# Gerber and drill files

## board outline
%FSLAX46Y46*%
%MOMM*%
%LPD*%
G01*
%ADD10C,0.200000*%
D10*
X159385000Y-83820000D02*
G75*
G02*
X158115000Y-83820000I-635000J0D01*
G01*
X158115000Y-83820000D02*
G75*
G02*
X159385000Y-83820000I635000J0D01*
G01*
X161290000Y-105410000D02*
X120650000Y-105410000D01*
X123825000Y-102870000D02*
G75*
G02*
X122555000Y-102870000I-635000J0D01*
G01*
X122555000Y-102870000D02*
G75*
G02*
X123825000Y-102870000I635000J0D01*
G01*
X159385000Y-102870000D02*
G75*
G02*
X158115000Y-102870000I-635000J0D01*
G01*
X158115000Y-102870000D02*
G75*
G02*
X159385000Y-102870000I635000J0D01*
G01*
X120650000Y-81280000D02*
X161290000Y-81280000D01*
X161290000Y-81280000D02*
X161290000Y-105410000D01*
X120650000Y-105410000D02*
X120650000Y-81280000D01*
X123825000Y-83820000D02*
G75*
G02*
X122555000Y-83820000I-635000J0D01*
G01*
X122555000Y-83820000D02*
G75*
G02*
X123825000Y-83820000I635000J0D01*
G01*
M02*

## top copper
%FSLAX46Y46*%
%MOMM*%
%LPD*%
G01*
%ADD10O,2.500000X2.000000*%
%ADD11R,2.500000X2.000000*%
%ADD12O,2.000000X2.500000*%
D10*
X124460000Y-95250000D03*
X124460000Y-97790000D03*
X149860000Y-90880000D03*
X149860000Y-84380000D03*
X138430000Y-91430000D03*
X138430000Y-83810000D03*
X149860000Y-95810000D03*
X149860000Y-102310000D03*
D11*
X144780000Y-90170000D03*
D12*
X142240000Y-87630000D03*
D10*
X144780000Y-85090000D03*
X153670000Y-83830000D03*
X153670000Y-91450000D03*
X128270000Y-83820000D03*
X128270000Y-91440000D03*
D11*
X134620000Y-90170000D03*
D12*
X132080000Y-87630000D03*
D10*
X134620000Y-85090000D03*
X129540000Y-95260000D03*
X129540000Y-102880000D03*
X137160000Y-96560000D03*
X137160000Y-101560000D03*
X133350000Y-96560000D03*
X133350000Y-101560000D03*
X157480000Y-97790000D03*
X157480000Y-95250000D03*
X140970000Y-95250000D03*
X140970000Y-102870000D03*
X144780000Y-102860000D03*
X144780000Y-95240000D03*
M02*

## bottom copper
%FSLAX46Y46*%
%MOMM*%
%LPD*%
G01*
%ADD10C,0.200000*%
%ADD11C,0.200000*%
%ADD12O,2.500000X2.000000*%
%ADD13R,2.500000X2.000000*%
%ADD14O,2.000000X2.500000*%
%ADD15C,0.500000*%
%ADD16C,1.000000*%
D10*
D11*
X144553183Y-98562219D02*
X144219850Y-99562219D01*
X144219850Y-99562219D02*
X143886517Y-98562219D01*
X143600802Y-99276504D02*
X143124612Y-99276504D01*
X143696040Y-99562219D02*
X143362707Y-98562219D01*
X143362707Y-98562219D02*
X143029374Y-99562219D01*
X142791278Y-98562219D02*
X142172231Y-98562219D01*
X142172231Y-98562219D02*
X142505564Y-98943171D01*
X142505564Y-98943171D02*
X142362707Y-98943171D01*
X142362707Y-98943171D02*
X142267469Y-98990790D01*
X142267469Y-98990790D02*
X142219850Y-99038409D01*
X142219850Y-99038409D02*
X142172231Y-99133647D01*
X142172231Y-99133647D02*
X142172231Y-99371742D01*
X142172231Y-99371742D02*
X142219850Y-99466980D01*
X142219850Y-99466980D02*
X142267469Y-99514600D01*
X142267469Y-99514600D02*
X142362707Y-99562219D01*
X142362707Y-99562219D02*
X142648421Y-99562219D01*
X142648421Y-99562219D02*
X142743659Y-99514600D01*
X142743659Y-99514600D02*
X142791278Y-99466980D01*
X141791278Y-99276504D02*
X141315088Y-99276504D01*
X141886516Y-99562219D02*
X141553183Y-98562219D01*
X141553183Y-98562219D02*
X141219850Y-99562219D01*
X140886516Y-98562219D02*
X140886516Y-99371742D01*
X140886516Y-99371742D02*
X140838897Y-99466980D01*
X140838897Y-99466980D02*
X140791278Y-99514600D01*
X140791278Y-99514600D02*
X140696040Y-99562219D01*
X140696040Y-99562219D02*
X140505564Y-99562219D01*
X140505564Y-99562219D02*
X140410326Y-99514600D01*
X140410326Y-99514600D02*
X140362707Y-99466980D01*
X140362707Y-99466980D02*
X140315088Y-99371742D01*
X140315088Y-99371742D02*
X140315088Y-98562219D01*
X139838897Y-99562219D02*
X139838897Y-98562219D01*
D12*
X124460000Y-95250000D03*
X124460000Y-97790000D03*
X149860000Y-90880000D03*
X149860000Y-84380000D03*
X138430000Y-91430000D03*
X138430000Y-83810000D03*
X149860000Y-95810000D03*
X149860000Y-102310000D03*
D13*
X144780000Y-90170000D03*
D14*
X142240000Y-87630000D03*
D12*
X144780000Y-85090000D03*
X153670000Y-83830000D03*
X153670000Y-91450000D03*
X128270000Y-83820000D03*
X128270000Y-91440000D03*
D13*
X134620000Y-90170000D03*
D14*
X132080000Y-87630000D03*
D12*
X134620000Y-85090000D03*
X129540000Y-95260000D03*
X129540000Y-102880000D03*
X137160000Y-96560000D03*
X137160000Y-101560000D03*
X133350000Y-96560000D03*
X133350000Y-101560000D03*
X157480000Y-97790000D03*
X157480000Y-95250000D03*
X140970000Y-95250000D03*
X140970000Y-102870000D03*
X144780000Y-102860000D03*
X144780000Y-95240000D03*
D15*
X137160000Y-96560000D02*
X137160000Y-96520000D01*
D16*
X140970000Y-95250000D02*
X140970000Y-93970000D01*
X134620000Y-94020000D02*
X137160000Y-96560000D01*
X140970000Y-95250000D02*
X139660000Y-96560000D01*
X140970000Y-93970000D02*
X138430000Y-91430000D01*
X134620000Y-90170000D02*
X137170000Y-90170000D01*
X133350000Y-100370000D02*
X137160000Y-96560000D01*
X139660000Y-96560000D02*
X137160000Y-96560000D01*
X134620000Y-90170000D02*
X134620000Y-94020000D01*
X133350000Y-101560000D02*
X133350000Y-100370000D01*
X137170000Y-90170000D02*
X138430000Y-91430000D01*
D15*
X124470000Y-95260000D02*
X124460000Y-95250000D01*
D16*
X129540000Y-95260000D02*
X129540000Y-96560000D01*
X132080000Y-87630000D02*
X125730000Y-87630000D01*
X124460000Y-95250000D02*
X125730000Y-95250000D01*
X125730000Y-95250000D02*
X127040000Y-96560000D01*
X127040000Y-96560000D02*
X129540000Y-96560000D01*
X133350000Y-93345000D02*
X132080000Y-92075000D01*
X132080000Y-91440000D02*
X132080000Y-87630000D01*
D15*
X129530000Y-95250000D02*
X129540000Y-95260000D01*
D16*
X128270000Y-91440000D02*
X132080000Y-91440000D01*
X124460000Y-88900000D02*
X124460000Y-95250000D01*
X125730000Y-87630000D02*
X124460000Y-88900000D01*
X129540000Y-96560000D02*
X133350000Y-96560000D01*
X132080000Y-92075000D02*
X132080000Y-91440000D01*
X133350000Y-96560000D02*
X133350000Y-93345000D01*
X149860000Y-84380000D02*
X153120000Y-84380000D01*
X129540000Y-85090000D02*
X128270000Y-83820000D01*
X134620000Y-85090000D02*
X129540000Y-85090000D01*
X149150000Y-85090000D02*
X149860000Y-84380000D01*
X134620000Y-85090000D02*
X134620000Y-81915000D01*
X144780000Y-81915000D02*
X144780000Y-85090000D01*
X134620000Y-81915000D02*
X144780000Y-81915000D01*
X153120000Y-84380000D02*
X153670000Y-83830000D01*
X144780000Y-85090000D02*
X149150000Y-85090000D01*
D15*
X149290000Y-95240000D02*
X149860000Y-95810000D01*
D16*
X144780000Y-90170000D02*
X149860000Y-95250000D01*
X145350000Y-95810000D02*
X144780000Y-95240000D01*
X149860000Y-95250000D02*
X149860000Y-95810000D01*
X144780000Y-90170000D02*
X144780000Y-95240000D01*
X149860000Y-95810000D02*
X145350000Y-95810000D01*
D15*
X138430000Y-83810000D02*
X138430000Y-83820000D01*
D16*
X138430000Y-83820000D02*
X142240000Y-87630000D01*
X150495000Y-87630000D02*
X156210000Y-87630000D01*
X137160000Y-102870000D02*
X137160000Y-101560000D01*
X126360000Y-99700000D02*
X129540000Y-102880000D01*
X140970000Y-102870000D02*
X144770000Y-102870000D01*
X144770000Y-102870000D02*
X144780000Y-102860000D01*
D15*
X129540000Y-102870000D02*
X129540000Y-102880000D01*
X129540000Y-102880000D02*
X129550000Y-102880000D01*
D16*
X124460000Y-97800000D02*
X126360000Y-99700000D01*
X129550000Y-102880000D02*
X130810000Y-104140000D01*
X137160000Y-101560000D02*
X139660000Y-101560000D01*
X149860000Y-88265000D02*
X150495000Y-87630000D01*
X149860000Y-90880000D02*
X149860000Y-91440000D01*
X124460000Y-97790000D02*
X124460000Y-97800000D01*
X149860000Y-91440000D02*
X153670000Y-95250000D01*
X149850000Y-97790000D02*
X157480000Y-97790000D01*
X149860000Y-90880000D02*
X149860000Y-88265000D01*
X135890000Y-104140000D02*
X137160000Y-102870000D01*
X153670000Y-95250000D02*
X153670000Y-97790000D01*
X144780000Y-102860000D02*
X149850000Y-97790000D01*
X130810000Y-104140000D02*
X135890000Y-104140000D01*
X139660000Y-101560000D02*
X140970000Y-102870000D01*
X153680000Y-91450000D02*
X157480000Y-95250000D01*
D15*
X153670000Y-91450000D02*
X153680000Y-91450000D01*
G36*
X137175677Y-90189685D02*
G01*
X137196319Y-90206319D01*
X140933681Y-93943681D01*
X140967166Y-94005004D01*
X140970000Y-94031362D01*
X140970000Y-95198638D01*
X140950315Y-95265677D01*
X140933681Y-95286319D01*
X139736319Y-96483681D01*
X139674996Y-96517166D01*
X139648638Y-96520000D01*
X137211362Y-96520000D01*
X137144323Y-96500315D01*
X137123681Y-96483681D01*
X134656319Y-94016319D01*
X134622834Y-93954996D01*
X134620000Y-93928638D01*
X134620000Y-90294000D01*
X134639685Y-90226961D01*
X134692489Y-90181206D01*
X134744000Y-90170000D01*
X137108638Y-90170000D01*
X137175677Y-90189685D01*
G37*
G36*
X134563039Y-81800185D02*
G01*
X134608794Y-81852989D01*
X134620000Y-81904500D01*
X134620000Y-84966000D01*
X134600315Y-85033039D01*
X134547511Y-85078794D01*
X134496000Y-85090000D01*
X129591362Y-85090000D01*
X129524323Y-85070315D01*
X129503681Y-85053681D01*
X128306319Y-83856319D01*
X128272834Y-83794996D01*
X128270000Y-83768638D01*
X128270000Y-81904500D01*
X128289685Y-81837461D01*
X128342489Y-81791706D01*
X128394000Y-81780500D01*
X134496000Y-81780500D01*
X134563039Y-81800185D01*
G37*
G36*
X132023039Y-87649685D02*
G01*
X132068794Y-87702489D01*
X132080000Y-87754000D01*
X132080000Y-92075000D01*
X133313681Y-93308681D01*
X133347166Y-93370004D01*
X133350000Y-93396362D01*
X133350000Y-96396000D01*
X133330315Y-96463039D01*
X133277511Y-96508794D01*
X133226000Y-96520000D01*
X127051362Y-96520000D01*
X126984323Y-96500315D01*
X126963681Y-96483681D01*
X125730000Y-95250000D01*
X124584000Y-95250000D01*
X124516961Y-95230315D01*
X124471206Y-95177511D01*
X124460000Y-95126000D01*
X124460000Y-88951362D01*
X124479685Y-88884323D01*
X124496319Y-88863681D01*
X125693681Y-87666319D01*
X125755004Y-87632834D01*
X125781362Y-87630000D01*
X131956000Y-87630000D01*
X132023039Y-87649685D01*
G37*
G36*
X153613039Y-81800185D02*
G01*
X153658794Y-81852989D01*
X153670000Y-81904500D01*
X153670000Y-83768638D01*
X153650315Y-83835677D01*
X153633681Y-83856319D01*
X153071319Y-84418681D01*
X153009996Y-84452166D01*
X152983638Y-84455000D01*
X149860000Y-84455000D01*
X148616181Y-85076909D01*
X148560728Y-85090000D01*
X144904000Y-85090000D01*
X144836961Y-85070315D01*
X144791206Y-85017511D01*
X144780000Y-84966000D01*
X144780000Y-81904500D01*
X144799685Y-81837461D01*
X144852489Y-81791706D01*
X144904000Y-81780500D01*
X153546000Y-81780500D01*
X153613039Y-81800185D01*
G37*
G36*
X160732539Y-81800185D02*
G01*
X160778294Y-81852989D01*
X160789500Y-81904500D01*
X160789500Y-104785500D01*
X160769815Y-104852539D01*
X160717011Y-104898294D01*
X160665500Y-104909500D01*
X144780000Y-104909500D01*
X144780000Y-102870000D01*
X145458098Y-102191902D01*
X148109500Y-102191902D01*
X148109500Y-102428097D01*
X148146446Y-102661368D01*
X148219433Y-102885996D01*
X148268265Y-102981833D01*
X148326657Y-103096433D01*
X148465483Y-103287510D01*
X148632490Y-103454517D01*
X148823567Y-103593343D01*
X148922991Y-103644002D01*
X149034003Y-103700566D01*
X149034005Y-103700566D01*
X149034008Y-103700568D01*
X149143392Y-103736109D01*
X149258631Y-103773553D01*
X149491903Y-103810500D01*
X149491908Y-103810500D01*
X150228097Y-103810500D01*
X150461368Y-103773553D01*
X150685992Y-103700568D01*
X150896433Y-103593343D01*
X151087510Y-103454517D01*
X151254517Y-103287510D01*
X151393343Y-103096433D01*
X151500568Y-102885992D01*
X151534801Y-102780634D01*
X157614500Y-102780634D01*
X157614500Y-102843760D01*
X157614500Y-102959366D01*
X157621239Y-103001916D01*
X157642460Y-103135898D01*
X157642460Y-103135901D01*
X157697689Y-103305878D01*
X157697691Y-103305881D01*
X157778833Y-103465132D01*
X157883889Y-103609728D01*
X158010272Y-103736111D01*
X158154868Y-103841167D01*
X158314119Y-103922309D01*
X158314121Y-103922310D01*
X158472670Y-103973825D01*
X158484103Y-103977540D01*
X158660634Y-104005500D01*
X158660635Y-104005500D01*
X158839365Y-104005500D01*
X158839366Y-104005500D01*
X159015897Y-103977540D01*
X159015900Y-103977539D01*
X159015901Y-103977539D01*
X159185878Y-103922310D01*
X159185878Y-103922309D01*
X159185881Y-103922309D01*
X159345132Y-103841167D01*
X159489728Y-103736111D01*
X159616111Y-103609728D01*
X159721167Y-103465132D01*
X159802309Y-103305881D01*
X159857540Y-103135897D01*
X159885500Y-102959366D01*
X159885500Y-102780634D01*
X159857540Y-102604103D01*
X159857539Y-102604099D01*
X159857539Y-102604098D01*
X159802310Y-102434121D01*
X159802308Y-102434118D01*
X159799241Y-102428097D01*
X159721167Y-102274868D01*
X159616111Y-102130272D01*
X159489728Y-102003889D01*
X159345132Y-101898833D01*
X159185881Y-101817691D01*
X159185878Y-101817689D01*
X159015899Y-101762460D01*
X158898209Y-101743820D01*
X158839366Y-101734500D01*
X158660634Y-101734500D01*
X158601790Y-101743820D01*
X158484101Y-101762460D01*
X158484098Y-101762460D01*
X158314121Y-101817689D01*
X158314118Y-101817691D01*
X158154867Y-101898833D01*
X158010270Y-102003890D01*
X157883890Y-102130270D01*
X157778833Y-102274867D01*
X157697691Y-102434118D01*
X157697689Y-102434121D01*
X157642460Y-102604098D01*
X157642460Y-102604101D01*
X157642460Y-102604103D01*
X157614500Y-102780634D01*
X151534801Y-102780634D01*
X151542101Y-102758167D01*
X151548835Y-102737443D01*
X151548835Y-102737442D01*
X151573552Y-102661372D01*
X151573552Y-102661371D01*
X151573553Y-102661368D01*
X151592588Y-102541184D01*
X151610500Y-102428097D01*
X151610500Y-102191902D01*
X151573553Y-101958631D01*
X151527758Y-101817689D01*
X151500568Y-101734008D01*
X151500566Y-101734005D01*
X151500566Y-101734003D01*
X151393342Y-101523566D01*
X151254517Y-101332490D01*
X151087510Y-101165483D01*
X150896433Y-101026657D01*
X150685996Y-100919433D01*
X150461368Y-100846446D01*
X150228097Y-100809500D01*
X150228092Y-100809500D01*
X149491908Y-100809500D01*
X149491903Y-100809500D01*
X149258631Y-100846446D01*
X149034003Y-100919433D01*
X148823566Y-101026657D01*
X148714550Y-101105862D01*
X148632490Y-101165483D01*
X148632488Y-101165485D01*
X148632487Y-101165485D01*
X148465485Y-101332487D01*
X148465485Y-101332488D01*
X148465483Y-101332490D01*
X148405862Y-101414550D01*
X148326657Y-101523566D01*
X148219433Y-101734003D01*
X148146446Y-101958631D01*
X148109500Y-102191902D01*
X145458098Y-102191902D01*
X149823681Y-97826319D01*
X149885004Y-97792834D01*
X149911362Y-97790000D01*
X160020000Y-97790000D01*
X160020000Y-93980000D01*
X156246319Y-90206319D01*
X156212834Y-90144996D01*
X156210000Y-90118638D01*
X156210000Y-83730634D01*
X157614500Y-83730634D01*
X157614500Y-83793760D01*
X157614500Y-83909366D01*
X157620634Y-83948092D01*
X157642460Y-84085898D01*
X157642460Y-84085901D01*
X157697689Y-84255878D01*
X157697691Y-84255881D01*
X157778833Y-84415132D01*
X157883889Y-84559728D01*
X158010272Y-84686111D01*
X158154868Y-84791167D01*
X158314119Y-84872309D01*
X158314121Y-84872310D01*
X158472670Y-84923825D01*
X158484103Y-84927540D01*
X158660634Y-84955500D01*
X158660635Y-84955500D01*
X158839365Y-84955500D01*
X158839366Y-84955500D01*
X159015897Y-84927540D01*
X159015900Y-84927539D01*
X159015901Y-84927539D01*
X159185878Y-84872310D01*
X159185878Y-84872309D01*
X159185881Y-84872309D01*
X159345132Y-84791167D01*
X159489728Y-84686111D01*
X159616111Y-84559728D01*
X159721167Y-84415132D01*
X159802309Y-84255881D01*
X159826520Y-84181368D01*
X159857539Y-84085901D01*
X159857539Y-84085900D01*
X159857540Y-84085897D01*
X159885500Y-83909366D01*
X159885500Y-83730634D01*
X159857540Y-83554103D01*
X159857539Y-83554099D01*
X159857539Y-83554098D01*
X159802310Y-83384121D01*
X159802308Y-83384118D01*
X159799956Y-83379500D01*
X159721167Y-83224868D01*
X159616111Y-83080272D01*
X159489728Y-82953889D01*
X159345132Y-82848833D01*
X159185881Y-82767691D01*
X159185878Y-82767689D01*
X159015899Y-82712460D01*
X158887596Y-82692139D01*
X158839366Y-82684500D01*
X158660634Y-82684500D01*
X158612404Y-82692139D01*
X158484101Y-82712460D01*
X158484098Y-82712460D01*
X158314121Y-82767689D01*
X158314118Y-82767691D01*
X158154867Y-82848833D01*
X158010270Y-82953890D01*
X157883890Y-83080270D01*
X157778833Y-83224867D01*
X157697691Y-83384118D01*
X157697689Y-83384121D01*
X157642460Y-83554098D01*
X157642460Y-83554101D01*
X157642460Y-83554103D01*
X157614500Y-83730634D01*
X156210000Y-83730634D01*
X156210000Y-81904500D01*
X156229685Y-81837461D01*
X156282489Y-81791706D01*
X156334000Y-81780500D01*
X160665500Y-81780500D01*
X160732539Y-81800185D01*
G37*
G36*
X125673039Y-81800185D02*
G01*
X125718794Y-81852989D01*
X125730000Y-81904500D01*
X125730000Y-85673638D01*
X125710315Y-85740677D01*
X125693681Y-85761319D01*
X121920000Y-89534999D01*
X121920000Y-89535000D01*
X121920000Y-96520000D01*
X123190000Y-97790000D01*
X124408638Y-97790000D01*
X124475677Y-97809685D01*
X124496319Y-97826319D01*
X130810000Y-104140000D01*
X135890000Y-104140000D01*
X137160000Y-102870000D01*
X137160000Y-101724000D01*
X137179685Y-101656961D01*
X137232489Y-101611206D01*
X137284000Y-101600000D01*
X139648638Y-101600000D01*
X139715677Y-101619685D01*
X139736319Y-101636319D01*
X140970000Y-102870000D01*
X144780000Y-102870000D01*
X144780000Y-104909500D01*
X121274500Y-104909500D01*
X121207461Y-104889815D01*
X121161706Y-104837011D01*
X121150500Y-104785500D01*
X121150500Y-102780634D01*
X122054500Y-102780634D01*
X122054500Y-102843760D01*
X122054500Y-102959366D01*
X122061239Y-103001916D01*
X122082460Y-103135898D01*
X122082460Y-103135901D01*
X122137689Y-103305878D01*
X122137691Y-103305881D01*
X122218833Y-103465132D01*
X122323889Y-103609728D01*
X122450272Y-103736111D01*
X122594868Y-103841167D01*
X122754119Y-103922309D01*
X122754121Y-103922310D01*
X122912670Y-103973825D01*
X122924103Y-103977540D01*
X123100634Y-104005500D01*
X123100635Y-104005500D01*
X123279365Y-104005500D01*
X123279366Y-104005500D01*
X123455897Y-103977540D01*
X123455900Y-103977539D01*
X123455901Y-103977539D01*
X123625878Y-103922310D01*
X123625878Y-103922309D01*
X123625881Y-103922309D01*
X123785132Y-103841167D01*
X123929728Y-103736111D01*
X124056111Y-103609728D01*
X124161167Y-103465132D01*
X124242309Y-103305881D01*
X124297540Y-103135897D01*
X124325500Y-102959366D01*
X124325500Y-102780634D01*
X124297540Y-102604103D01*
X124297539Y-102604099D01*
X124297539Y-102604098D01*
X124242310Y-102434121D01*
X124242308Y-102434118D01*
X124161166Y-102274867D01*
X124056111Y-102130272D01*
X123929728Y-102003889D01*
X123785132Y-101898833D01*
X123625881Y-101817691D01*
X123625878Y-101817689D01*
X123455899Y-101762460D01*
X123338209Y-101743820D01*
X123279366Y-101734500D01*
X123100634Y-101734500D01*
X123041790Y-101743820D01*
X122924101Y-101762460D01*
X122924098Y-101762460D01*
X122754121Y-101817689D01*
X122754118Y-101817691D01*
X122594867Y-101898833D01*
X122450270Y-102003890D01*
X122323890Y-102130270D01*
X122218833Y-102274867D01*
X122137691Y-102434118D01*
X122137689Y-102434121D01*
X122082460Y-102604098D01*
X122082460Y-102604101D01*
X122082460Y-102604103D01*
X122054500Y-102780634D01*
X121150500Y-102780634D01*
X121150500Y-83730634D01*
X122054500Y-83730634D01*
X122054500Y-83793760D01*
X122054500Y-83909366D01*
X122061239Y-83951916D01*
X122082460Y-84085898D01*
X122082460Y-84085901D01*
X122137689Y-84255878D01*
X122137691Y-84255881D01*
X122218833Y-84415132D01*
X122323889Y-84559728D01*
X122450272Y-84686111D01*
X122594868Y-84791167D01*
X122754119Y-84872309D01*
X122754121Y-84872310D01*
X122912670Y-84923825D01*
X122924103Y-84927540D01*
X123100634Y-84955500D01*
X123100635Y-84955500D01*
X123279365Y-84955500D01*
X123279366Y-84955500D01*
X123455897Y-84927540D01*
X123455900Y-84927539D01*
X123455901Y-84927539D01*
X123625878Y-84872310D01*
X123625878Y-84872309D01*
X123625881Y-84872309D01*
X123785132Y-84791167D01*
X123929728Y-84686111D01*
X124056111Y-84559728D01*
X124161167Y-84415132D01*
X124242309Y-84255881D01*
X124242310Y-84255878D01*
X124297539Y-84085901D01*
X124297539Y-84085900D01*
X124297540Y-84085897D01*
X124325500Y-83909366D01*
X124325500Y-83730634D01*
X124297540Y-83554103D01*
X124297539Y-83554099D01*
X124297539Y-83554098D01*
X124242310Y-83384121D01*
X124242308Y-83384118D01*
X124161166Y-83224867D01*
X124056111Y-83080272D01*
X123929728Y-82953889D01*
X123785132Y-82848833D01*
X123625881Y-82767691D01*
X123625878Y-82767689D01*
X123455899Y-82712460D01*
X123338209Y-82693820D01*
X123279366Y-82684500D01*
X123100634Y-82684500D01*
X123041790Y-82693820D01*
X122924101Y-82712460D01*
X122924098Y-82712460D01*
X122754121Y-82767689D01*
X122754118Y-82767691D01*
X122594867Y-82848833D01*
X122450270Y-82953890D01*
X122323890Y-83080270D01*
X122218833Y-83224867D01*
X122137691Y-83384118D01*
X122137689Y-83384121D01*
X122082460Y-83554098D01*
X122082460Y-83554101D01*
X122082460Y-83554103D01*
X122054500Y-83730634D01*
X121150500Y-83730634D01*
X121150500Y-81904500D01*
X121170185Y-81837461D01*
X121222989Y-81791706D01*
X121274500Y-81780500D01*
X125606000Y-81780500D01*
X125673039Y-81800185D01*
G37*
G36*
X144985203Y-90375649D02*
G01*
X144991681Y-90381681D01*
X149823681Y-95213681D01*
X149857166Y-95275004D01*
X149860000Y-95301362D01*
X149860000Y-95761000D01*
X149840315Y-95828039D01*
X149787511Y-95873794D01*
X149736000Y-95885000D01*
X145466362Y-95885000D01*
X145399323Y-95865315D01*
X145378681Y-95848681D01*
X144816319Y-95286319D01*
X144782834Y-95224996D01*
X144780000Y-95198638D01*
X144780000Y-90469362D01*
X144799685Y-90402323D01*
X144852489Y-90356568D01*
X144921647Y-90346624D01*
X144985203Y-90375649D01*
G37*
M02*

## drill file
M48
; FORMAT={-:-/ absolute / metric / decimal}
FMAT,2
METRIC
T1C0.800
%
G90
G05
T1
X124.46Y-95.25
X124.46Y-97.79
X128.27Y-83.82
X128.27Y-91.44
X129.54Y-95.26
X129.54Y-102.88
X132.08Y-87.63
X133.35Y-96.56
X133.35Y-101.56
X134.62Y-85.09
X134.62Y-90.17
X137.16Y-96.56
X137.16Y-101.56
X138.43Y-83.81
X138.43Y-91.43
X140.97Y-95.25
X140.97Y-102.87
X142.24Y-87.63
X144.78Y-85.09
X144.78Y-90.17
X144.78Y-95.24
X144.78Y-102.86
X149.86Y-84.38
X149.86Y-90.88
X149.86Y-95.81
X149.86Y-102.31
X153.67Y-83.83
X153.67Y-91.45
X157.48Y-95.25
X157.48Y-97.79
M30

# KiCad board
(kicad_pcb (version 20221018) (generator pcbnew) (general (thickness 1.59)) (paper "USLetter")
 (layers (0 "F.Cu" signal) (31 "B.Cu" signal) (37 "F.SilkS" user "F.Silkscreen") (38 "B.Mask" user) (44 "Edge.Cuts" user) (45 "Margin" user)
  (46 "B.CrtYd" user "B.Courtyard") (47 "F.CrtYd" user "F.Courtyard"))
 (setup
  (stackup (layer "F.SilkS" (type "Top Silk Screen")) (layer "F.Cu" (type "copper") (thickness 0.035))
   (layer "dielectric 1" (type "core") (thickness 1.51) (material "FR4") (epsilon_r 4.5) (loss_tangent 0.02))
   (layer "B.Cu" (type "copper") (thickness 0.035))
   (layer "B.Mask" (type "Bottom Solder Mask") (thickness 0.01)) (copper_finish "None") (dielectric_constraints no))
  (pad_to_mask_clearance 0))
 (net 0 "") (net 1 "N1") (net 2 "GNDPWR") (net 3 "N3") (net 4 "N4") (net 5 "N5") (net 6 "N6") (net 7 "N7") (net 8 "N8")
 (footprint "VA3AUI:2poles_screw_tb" (layer "F.Cu") (at 124.46 96.52 -90)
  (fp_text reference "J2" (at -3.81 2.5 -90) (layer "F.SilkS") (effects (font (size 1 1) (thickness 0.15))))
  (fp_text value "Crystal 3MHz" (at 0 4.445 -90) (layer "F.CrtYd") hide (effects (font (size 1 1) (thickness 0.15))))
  (pad "1" thru_hole oval (at -1.27 0 270) (size 2 2.5) (drill 0.8) (layers "*.Cu") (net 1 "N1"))
  (pad "2" thru_hole oval (at 1.27 0 270) (size 2 2.5) (drill 0.8) (layers "*.Cu") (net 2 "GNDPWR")))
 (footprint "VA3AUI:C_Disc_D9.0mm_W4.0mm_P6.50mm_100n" (layer "F.Cu") (at 149.86 87.63 90)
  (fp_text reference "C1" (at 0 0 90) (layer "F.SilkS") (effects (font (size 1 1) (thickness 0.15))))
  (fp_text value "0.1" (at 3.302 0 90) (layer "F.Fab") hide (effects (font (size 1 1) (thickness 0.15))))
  (pad "1" thru_hole oval (at -3.25 0 90) (size 2 2.5) (drill 0.8) (layers "*.Cu") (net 2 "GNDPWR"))
  (pad "2" thru_hole oval (at 3.25 0 90) (size 2 2.5) (drill 0.8) (layers "*.Cu") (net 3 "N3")))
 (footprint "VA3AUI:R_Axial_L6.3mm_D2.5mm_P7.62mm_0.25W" (layer "F.Cu") (at 138.43 91.43 90)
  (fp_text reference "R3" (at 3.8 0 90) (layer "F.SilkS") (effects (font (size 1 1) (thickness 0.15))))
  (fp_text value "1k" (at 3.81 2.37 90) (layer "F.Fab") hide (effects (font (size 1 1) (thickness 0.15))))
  (pad "1" thru_hole oval (at 0 0 90) (size 2 2.5) (drill 0.8) (layers "*.Cu") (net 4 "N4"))
  (pad "2" thru_hole oval (at 7.62 0 90) (size 2 2.5) (drill 0.8) (layers "*.Cu") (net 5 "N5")))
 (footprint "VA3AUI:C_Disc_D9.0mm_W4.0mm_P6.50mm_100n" (layer "F.Cu") (at 149.86 99.06 -90)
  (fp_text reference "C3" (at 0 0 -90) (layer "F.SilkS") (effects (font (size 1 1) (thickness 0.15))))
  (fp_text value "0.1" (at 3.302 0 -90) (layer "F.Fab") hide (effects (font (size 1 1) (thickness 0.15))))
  (pad "1" thru_hole oval (at -3.25 0 270) (size 2 2.5) (drill 0.8) (layers "*.Cu") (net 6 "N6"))
  (pad "2" thru_hole oval (at 3.25 0 270) (size 2 2.5) (drill 0.8) (layers "*.Cu") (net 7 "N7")))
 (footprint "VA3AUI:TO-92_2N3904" (layer "F.Cu") (at 144.78 87.63 90)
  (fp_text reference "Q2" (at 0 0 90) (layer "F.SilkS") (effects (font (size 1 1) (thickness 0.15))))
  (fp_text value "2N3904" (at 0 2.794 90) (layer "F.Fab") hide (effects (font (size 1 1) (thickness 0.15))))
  (pad "1" thru_hole rect (at -2.54 0 90) (size 2 2.5) (drill 0.8) (layers "*.Cu") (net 6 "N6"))
  (pad "2" thru_hole oval (at 0 -2.54 90) (size 2.5 2) (drill 0.8) (layers "*.Cu") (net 5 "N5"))
  (pad "3" thru_hole oval (at 2.54 0 90) (size 2 2.5) (drill 0.8) (layers "*.Cu") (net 3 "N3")))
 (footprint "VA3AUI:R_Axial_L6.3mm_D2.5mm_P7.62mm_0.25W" (layer "F.Cu") (at 153.67 83.83 -90)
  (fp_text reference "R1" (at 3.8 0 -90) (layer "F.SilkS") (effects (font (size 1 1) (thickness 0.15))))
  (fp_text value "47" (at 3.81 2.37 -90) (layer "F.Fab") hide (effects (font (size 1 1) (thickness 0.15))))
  (pad "1" thru_hole oval (at 0 0 270) (size 2 2.5) (drill 0.8) (layers "*.Cu") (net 3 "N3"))
  (pad "2" thru_hole oval (at 7.62 0 270) (size 2 2.5) (drill 0.8) (layers "*.Cu") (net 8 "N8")))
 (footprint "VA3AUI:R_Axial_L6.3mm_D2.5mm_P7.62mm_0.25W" (layer "F.Cu") (at 128.27 83.82 -90)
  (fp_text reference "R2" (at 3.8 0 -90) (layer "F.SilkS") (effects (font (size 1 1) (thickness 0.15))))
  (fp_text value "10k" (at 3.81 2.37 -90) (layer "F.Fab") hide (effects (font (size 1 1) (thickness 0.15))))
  (pad "1" thru_hole oval (at 0 0 270) (size 2 2.5) (drill 0.8) (layers "*.Cu") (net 3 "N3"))
  (pad "2" thru_hole oval (at 7.62 0 270) (size 2 2.5) (drill 0.8) (layers "*.Cu") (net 1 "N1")))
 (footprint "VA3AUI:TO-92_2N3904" (layer "F.Cu") (at 134.62 87.63 90)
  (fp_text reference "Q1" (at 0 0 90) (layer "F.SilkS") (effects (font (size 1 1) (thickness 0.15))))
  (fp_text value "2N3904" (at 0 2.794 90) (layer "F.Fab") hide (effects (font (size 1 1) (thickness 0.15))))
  (pad "1" thru_hole rect (at -2.54 0 90) (size 2 2.5) (drill 0.8) (layers "*.Cu") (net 4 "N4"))
  (pad "2" thru_hole oval (at 0 -2.54 90) (size 2.5 2) (drill 0.8) (layers "*.Cu") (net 1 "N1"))
  (pad "3" thru_hole oval (at 2.54 0 90) (size 2 2.5) (drill 0.8) (layers "*.Cu") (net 3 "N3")))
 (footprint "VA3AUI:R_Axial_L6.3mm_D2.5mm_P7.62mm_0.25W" (layer "F.Cu") (at 129.54 95.26 -90)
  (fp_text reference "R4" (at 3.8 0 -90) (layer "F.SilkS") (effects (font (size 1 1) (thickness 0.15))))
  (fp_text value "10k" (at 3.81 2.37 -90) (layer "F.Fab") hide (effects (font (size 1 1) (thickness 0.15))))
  (pad "1" thru_hole oval (at 0 0 270) (size 2 2.5) (drill 0.8) (layers "*.Cu") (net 1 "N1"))
  (pad "2" thru_hole oval (at 7.62 0 270) (size 2 2.5) (drill 0.8) (layers "*.Cu") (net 2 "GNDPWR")))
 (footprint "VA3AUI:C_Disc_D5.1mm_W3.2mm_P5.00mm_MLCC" (layer "F.Cu") (at 137.16 96.56 -90)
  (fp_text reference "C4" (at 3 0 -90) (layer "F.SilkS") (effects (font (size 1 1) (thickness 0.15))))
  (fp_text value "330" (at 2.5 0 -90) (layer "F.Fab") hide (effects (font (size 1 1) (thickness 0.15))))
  (pad "1" thru_hole oval (at 0 0 270) (size 2 2.5) (drill 0.8) (layers "*.Cu") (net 4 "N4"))
  (pad "2" thru_hole oval (at 5 0 270) (size 2 2.5) (drill 0.8) (layers "*.Cu") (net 2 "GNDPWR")))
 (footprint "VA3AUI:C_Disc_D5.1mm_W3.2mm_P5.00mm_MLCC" (layer "F.Cu") (at 133.35 96.56 -90)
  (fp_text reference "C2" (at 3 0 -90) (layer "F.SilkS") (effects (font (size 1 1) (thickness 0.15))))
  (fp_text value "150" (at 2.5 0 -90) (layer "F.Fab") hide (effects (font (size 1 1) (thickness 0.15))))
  (pad "1" thru_hole oval (at 0 0 270) (size 2 2.5) (drill 0.8) (layers "*.Cu") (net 1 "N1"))
  (pad "2" thru_hole oval (at 5 0 270) (size 2 2.5) (drill 0.8) (layers "*.Cu") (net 4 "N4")))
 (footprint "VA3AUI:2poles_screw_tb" (layer "F.Cu") (at 157.48 96.52 90)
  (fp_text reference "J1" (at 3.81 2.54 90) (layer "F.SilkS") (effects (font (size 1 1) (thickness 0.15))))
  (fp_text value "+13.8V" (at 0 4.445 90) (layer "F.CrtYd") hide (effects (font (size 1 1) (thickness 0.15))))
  (pad "1" thru_hole oval (at -1.27 0 90) (size 2 2.5) (drill 0.8) (layers "*.Cu") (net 2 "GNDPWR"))
  (pad "2" thru_hole oval (at 1.27 0 90) (size 2 2.5) (drill 0.8) (layers "*.Cu") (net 8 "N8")))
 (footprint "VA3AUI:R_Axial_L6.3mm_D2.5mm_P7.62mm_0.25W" (layer "F.Cu") (at 140.97 95.25 -90)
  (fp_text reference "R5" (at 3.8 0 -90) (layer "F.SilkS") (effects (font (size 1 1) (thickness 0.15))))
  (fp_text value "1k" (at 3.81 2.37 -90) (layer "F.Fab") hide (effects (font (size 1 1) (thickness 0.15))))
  (pad "1" thru_hole oval (at 0 0 270) (size 2 2.5) (drill 0.8) (layers "*.Cu") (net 4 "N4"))
  (pad "2" thru_hole oval (at 7.62 0 270) (size 2 2.5) (drill 0.8) (layers "*.Cu") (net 2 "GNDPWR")))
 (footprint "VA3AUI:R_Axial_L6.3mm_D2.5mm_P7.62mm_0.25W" (layer "F.Cu") (at 144.78 102.86 90)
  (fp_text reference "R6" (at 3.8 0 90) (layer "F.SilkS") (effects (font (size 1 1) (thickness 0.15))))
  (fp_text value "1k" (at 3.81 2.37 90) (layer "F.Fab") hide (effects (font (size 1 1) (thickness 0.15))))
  (pad "1" thru_hole oval (at 0 0 90) (size 2 2.5) (drill 0.8) (layers "*.Cu") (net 2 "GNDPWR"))
  (pad "2" thru_hole oval (at 7.62 0 90) (size 2 2.5) (drill 0.8) (layers "*.Cu") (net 6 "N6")))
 (gr_circle (center 158.75 83.82) (end 159.385 83.82) (stroke (width 0.2) (type default)) (fill none) (layer "Edge.Cuts"))
 (gr_line (start 161.29 105.41) (end 120.65 105.41) (stroke (width 0.2) (type default)) (layer "Edge.Cuts"))
 (gr_circle (center 123.19 102.87) (end 123.825 102.87) (stroke (width 0.2) (type default)) (fill none) (layer "Edge.Cuts"))
 (gr_circle (center 158.75 102.87) (end 159.385 102.87) (stroke (width 0.2) (type default)) (fill none) (layer "Edge.Cuts"))
 (gr_line (start 120.65 81.28) (end 161.29 81.28) (stroke (width 0.2) (type default)) (layer "Edge.Cuts"))
 (gr_line (start 161.29 81.28) (end 161.29 105.41) (stroke (width 0.2) (type default)) (layer "Edge.Cuts"))
 (gr_line (start 120.65 105.41) (end 120.65 81.28) (stroke (width 0.2) (type default)) (layer "Edge.Cuts"))
 (gr_circle (center 123.19 83.82) (end 123.825 83.82) (stroke (width 0.2) (type default)) (fill none) (layer "Edge.Cuts"))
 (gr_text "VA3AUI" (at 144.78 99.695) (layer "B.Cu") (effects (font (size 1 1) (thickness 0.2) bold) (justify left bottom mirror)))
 (segment (start 137.16 96.56) (end 137.16 96.52) (width 0.5) (layer "B.Cu") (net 4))
 (segment (start 140.97 95.25) (end 140.97 93.97) (width 1) (layer "B.Cu") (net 4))
 (segment (start 134.62 94.02) (end 137.16 96.56) (width 1) (layer "B.Cu") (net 4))
 (segment (start 140.97 95.25) (end 139.66 96.56) (width 1) (layer "B.Cu") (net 4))
 (segment (start 140.97 93.97) (end 138.43 91.43) (width 1) (layer "B.Cu") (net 4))
 (segment (start 134.62 90.17) (end 137.17 90.17) (width 1) (layer "B.Cu") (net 4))
 (segment (start 133.35 100.37) (end 137.16 96.56) (width 1) (layer "B.Cu") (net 4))
 (segment (start 139.66 96.56) (end 137.16 96.56) (width 1) (layer "B.Cu") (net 4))
 (segment (start 134.62 90.17) (end 134.62 94.02) (width 1) (layer "B.Cu") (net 4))
 (segment (start 133.35 101.56) (end 133.35 100.37) (width 1) (layer "B.Cu") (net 4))
 (segment (start 137.17 90.17) (end 138.43 91.43) (width 1) (layer "B.Cu") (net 4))
 (segment (start 124.47 95.26) (end 124.46 95.25) (width 0.5) (layer "B.Cu") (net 1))
 (segment (start 129.54 95.26) (end 129.54 96.56) (width 1) (layer "B.Cu") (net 1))
 (segment (start 132.08 87.63) (end 125.73 87.63) (width 1) (layer "B.Cu") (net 1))
 (segment (start 124.46 95.25) (end 125.73 95.25) (width 1) (layer "B.Cu") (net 1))
 (segment (start 125.73 95.25) (end 127.04 96.56) (width 1) (layer "B.Cu") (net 1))
 (segment (start 127.04 96.56) (end 129.54 96.56) (width 1) (layer "B.Cu") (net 1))
 (segment (start 133.35 93.345) (end 132.08 92.075) (width 1) (layer "B.Cu") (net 1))
 (segment (start 132.08 91.44) (end 132.08 87.63) (width 1) (layer "B.Cu") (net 1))
 (segment (start 129.53 95.25) (end 129.54 95.26) (width 0.5) (layer "B.Cu") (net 1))
 (segment (start 128.27 91.44) (end 132.08 91.44) (width 1) (layer "B.Cu") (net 1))
 (segment (start 124.46 88.9) (end 124.46 95.25) (width 1) (layer "B.Cu") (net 1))
 (segment (start 125.73 87.63) (end 124.46 88.9) (width 1) (layer "B.Cu") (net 1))
 (segment (start 129.54 96.56) (end 133.35 96.56) (width 1) (layer "B.Cu") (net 1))
 (segment (start 132.08 92.075) (end 132.08 91.44) (width 1) (layer "B.Cu") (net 1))
 (segment (start 133.35 96.56) (end 133.35 93.345) (width 1) (layer "B.Cu") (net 1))
 (segment (start 149.86 84.38) (end 153.12 84.38) (width 1) (layer "B.Cu") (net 3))
 (segment (start 129.54 85.09) (end 128.27 83.82) (width 1) (layer "B.Cu") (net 3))
 (segment (start 134.62 85.09) (end 129.54 85.09) (width 1) (layer "B.Cu") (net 3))
 (segment (start 149.15 85.09) (end 149.86 84.38) (width 1) (layer "B.Cu") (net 3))
 (segment (start 134.62 85.09) (end 134.62 81.915) (width 1) (layer "B.Cu") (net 3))
 (segment (start 144.78 81.915) (end 144.78 85.09) (width 1) (layer "B.Cu") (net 3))
 (segment (start 134.62 81.915) (end 144.78 81.915) (width 1) (layer "B.Cu") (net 3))
 (segment (start 153.12 84.38) (end 153.67 83.83) (width 1) (layer "B.Cu") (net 3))
 (segment (start 144.78 85.09) (end 149.15 85.09) (width 1) (layer "B.Cu") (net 3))
 (segment (start 149.29 95.24) (end 149.86 95.81) (width 0.5) (layer "B.Cu") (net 6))
 (segment (start 144.78 90.17) (end 149.86 95.25) (width 1) (layer "B.Cu") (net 6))
 (segment (start 145.35 95.81) (end 144.78 95.24) (width 1) (layer "B.Cu") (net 6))
 (segment (start 149.86 95.25) (end 149.86 95.81) (width 1) (layer "B.Cu") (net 6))
 (segment (start 144.78 90.17) (end 144.78 95.24) (width 1) (layer "B.Cu") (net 6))
 (segment (start 149.86 95.81) (end 145.35 95.81) (width 1) (layer "B.Cu") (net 6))
 (segment (start 138.43 83.81) (end 138.43 83.82) (width 0.5) (layer "B.Cu") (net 5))
 (segment (start 138.43 83.82) (end 142.24 87.63) (width 1) (layer "B.Cu") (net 5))
 (segment (start 150.495 87.63) (end 156.21 87.63) (width 1) (layer "B.Cu") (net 2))
 (segment (start 137.16 102.87) (end 137.16 101.56) (width 1) (layer "B.Cu") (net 2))
 (segment (start 126.36 99.7) (end 129.54 102.88) (width 1) (layer "B.Cu") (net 2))
 (segment (start 140.97 102.87) (end 144.77 102.87) (width 1) (layer "B.Cu") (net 2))
 (segment (start 144.77 102.87) (end 144.78 102.86) (width 1) (layer "B.Cu") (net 2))
 (segment (start 129.54 102.87) (end 129.54 102.88) (width 0.5) (layer "B.Cu") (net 2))
 (segment (start 129.54 102.88) (end 129.55 102.88) (width 0.5) (layer "B.Cu") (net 2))
 (segment (start 124.46 97.8) (end 126.36 99.7) (width 1) (layer "B.Cu") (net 2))
 (segment (start 129.55 102.88) (end 130.81 104.14) (width 1) (layer "B.Cu") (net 2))
 (segment (start 137.16 101.56) (end 139.66 101.56) (width 1) (layer "B.Cu") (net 2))
 (segment (start 149.86 88.265) (end 150.495 87.63) (width 1) (layer "B.Cu") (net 2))
 (segment (start 149.86 90.88) (end 149.86 91.44) (width 1) (layer "B.Cu") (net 2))
 (segment (start 124.46 97.79) (end 124.46 97.8) (width 1) (layer "B.Cu") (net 2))
 (segment (start 149.86 91.44) (end 153.67 95.25) (width 1) (layer "B.Cu") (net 2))
 (segment (start 149.85 97.79) (end 157.48 97.79) (width 1) (layer "B.Cu") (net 2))
 (segment (start 149.86 90.88) (end 149.86 88.265) (width 1) (layer "B.Cu") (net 2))
 (segment (start 135.89 104.14) (end 137.16 102.87) (width 1) (layer "B.Cu") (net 2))
 (segment (start 153.67 95.25) (end 153.67 97.79) (width 1) (layer "B.Cu") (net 2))
 (segment (start 144.78 102.86) (end 149.85 97.79) (width 1) (layer "B.Cu") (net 2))
 (segment (start 130.81 104.14) (end 135.89 104.14) (width 1) (layer "B.Cu") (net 2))
 (segment (start 139.66 101.56) (end 140.97 102.87) (width 1) (layer "B.Cu") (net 2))
 (segment (start 153.68 91.45) (end 157.48 95.25) (width 1) (layer "B.Cu") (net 8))
 (segment (start 153.67 91.45) (end 153.68 91.45) (width 0.5) (layer "B.Cu") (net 8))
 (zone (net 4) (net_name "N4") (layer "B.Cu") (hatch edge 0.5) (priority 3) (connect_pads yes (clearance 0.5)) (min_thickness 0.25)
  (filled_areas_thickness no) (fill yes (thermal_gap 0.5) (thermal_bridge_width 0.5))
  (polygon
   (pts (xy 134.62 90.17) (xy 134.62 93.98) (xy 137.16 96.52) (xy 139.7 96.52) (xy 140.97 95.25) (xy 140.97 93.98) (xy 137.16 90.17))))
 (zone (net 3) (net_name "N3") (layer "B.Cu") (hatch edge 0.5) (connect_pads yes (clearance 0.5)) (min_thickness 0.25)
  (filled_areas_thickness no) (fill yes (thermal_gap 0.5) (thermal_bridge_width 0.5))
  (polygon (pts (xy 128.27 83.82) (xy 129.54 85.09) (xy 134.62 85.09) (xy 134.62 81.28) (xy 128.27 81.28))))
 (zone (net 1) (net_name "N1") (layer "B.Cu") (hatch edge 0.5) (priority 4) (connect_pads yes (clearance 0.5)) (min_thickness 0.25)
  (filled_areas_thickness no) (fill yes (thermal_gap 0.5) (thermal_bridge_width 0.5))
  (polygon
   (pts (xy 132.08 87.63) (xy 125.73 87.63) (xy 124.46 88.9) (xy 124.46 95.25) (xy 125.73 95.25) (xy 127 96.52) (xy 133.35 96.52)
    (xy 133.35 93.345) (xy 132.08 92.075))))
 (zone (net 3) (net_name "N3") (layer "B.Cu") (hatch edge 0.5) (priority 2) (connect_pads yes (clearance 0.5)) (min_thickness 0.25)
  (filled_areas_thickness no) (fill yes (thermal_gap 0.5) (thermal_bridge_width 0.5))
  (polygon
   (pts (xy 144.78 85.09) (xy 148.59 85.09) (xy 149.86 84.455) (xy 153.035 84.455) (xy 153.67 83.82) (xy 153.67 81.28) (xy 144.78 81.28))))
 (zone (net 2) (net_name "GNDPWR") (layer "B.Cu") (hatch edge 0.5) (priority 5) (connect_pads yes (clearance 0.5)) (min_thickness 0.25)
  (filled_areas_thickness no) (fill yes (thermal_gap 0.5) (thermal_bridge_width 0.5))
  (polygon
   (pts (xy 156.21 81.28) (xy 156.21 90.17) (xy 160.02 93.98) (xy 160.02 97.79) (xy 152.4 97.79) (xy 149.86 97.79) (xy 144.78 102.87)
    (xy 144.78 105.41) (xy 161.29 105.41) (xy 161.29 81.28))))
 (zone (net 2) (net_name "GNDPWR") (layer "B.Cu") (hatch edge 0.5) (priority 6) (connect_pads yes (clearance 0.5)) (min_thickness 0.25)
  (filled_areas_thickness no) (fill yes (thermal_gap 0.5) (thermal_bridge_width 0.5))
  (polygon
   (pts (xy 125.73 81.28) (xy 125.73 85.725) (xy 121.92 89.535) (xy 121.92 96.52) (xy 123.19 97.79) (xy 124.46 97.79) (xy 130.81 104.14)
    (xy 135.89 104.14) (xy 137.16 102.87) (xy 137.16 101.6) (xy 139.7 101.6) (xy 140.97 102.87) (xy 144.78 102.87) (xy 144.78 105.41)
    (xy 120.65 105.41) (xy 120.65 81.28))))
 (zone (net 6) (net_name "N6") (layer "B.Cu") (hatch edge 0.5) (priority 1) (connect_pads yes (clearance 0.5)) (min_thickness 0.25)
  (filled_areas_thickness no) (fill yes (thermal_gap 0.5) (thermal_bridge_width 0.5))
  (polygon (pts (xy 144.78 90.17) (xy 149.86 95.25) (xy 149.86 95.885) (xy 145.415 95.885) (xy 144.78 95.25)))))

